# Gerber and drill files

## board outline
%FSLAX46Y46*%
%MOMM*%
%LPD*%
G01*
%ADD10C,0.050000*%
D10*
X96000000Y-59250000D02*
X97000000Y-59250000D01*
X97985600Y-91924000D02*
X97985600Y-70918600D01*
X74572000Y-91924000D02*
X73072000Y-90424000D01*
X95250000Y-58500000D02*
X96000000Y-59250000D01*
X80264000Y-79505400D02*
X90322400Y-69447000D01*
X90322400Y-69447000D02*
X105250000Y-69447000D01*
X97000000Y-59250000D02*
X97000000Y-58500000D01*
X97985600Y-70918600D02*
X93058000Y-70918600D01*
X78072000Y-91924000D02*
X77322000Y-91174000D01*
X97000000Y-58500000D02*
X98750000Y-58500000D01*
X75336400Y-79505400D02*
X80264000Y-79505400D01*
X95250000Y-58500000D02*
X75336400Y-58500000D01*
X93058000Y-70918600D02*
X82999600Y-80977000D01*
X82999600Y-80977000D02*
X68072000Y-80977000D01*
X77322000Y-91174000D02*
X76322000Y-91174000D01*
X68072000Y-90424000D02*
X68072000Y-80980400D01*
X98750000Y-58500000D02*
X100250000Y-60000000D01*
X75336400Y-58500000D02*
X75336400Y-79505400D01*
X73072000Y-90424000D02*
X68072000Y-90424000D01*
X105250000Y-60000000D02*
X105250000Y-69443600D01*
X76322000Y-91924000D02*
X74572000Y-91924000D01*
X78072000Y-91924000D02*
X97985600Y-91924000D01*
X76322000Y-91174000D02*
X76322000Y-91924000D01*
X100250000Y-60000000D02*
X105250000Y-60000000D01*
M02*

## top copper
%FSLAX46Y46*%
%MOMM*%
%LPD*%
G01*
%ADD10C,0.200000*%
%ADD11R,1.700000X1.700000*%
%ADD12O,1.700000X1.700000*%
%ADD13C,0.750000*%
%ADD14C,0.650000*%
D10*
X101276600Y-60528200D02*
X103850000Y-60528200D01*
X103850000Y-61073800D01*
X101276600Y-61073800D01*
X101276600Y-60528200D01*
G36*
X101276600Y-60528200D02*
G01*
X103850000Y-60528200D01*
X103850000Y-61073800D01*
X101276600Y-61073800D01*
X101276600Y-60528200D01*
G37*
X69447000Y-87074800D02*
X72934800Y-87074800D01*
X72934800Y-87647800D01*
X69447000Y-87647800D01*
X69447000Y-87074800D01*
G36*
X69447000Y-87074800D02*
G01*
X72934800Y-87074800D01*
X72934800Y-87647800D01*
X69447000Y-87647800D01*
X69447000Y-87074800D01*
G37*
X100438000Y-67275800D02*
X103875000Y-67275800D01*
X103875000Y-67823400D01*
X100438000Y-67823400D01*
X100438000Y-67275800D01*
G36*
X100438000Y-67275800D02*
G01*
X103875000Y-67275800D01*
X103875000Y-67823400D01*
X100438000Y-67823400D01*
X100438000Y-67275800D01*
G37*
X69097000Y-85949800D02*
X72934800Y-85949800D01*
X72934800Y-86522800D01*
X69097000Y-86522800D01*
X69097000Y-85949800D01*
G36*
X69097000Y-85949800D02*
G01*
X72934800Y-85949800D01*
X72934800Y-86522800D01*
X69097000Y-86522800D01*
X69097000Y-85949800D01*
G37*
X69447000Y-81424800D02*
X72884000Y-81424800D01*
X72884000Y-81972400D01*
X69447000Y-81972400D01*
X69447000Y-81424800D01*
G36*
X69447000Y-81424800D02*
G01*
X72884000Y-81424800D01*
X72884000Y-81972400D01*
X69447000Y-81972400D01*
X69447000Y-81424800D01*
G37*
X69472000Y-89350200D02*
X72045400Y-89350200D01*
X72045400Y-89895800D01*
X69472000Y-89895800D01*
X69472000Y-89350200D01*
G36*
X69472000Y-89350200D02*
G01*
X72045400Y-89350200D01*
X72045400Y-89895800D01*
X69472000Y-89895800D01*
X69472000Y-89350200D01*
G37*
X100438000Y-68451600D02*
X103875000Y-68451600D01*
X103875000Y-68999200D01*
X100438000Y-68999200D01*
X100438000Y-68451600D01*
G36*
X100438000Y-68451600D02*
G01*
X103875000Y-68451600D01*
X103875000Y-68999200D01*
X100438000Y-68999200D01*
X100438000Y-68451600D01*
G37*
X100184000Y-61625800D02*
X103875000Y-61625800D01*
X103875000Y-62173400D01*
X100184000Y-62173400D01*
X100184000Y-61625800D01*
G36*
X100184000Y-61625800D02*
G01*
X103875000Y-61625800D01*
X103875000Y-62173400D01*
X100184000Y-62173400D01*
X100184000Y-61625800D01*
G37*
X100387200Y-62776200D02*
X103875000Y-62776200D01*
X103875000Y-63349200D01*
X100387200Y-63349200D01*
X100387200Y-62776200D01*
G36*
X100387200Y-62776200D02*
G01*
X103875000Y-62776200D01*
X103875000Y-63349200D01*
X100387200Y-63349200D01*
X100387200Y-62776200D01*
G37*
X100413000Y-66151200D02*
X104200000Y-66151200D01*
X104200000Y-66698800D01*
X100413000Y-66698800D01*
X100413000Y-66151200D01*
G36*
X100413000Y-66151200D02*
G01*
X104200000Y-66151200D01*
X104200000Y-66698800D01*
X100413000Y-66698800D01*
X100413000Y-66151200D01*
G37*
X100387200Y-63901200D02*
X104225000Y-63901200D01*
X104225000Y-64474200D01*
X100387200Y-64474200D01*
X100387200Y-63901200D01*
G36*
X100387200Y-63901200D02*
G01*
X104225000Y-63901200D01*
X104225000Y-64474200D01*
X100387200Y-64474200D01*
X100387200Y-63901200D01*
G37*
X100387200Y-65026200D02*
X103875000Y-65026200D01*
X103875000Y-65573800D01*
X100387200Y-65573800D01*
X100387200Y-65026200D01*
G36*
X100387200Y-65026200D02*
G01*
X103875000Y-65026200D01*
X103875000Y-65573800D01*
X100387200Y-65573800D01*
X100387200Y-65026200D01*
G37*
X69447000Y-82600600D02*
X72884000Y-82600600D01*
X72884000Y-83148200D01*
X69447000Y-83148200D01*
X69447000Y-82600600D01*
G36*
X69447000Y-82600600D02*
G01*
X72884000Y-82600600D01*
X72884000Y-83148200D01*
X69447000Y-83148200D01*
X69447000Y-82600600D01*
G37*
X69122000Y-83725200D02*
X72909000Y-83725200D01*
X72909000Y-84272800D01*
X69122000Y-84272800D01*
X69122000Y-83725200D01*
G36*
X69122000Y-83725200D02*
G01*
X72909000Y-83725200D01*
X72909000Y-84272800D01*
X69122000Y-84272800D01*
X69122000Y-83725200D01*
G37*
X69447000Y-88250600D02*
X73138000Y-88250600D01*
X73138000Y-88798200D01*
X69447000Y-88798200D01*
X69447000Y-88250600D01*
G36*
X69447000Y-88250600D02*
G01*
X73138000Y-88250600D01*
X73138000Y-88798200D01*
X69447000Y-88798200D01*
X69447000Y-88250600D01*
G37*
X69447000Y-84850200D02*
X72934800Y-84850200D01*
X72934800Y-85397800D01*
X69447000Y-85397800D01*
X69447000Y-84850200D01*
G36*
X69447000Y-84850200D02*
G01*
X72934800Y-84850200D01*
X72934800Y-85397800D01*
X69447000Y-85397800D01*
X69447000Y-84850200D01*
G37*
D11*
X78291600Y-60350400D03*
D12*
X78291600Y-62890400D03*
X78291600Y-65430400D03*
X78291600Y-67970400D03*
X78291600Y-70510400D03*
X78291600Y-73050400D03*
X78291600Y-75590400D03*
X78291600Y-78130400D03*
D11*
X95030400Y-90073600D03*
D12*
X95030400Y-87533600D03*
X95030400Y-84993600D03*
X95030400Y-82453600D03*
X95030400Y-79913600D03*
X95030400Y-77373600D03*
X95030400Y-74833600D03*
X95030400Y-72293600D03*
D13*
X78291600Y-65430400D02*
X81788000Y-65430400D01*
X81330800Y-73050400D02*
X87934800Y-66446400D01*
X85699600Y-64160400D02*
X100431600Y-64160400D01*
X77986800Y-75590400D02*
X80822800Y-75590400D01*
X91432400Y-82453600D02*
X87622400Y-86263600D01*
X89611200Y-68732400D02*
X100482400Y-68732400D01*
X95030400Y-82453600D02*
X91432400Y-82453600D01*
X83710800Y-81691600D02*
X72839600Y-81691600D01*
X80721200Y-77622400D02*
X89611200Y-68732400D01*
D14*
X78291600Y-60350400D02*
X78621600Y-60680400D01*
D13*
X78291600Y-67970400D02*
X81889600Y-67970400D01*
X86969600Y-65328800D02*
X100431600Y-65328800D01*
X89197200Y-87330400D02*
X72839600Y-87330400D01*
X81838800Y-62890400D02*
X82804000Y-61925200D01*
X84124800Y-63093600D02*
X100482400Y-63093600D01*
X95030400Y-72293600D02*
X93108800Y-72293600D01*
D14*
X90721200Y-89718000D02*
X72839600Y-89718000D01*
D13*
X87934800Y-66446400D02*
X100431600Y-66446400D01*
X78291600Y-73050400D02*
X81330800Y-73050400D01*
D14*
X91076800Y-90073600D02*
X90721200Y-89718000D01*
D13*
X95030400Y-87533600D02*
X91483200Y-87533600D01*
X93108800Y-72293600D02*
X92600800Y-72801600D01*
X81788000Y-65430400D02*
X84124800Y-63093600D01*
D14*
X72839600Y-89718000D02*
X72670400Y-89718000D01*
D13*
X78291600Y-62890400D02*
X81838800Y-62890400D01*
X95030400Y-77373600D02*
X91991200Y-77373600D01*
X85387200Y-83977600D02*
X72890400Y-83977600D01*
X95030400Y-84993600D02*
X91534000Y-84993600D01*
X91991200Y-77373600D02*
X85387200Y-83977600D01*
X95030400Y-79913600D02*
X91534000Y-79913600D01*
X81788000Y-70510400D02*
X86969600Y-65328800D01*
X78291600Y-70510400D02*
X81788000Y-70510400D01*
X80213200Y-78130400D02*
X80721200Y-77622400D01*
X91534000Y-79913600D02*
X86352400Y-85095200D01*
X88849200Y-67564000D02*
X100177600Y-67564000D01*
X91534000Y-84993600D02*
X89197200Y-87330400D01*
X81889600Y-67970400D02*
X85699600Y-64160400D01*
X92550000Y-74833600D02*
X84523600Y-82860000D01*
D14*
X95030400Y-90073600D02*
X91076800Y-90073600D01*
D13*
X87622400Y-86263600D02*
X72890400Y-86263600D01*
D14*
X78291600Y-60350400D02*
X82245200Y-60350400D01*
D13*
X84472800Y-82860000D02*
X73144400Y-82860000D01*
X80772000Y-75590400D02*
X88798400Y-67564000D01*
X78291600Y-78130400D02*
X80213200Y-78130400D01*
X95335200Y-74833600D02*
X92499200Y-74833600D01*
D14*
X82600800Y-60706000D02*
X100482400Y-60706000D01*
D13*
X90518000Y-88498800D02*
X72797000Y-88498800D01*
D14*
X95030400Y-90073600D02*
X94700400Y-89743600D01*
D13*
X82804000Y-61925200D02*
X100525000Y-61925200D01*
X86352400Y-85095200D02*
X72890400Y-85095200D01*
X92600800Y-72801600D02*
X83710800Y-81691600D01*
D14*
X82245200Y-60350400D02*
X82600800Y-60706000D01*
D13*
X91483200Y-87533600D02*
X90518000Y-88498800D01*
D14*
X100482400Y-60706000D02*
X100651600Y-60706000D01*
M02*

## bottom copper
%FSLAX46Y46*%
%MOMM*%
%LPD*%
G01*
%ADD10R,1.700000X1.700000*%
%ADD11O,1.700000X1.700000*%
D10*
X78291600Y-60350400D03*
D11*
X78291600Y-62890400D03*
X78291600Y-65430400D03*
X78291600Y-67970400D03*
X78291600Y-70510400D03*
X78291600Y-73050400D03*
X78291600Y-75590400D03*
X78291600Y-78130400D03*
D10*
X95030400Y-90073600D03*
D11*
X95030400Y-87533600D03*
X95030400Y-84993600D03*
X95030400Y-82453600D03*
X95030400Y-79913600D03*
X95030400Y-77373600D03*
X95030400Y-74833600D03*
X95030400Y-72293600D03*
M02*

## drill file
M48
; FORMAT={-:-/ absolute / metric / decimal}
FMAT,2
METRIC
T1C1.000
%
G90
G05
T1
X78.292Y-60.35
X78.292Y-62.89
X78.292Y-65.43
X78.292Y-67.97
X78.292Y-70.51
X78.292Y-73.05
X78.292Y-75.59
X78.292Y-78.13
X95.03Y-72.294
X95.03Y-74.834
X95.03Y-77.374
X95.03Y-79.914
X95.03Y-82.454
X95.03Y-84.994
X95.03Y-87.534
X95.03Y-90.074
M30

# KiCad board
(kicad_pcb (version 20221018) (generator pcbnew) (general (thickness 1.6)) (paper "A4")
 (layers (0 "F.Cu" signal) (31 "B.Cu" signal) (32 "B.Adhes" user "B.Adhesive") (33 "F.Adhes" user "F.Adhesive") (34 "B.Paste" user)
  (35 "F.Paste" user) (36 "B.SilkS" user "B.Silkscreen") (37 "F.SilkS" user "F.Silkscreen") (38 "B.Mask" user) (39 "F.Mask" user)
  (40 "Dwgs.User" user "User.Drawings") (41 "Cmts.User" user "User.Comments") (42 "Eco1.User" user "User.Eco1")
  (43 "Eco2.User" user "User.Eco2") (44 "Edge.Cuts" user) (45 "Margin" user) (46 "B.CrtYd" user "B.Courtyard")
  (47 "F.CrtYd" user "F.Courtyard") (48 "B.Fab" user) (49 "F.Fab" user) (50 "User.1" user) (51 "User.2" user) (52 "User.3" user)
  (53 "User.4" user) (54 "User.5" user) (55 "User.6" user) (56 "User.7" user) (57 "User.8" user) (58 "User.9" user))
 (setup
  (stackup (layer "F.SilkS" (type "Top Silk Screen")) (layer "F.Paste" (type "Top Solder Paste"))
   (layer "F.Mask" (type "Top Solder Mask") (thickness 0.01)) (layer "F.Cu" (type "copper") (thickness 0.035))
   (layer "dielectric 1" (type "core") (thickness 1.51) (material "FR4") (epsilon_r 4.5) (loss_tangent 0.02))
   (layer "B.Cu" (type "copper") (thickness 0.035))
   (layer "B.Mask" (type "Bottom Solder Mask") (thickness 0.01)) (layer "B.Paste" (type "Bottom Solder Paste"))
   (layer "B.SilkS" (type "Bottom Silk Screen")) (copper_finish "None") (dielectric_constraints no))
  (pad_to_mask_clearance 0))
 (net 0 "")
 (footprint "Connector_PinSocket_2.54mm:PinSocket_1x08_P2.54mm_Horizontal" (layer "F.Cu") (at 78.2916 60.3504)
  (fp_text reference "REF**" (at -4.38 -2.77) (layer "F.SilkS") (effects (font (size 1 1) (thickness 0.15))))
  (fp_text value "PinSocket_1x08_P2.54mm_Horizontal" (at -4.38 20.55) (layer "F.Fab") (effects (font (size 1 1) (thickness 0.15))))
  (pad "1" thru_hole rect (at 0 0) (size 1.7 1.7) (drill 1) (layers "*.Cu" "*.Mask"))
  (pad "2" thru_hole oval (at 0 2.54) (size 1.7 1.7) (drill 1) (layers "*.Cu" "*.Mask"))
  (pad "3" thru_hole oval (at 0 5.08) (size 1.7 1.7) (drill 1) (layers "*.Cu" "*.Mask"))
  (pad "4" thru_hole oval (at 0 7.62) (size 1.7 1.7) (drill 1) (layers "*.Cu" "*.Mask"))
  (pad "5" thru_hole oval (at 0 10.16) (size 1.7 1.7) (drill 1) (layers "*.Cu" "*.Mask"))
  (pad "6" thru_hole oval (at 0 12.7) (size 1.7 1.7) (drill 1) (layers "*.Cu" "*.Mask"))
  (pad "7" thru_hole oval (at 0 15.24) (size 1.7 1.7) (drill 1) (layers "*.Cu" "*.Mask"))
  (pad "8" thru_hole oval (at 0 17.78) (size 1.7 1.7) (drill 1) (layers "*.Cu" "*.Mask")))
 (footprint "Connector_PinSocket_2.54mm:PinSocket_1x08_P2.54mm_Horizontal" (layer "F.Cu") (at 95.0304 90.0736 180)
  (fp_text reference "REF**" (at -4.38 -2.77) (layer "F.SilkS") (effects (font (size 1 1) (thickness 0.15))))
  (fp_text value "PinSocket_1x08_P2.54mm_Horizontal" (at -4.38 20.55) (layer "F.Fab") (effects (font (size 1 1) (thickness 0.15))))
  (pad "1" thru_hole rect (at 0 0 180) (size 1.7 1.7) (drill 1) (layers "*.Cu" "*.Mask"))
  (pad "2" thru_hole oval (at 0 2.54 180) (size 1.7 1.7) (drill 1) (layers "*.Cu" "*.Mask"))
  (pad "3" thru_hole oval (at 0 5.08 180) (size 1.7 1.7) (drill 1) (layers "*.Cu" "*.Mask"))
  (pad "4" thru_hole oval (at 0 7.62 180) (size 1.7 1.7) (drill 1) (layers "*.Cu" "*.Mask"))
  (pad "5" thru_hole oval (at 0 10.16 180) (size 1.7 1.7) (drill 1) (layers "*.Cu" "*.Mask"))
  (pad "6" thru_hole oval (at 0 12.7 180) (size 1.7 1.7) (drill 1) (layers "*.Cu" "*.Mask"))
  (pad "7" thru_hole oval (at 0 15.24 180) (size 1.7 1.7) (drill 1) (layers "*.Cu" "*.Mask"))
  (pad "8" thru_hole oval (at 0 17.78 180) (size 1.7 1.7) (drill 1) (layers "*.Cu" "*.Mask")))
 (gr_rect (start 101.2766 60.5282) (end 103.85 61.0738) (stroke (width 0.2) (type solid)) (fill solid) (layer "F.Cu"))
 (gr_rect (start 72.9348 87.6478) (end 69.447 87.0748) (stroke (width 0.2) (type solid)) (fill solid) (layer "F.Cu"))
 (gr_rect (start 100.438 67.2758) (end 103.875 67.8234) (stroke (width 0.2) (type solid)) (fill solid) (layer "F.Cu"))
 (gr_rect (start 72.9348 86.5228) (end 69.097 85.9498) (stroke (width 0.2) (type solid)) (fill solid) (layer "F.Cu"))
 (gr_rect (start 72.884 81.9724) (end 69.447 81.4248) (stroke (width 0.2) (type solid)) (fill solid) (layer "F.Cu"))
 (gr_rect (start 72.0454 89.8958) (end 69.472 89.3502) (stroke (width 0.2) (type solid)) (fill solid) (layer "F.Cu"))
 (gr_rect (start 100.438 68.4516) (end 103.875 68.9992) (stroke (width 0.2) (type solid)) (fill solid) (layer "F.Cu"))
 (gr_rect (start 100.184 61.6258) (end 103.875 62.1734) (stroke (width 0.2) (type solid)) (fill solid) (layer "F.Cu"))
 (gr_rect (start 100.3872 62.7762) (end 103.875 63.3492) (stroke (width 0.2) (type solid)) (fill solid) (layer "F.Cu"))
 (gr_rect (start 100.413 66.1512) (end 104.2 66.6988) (stroke (width 0.2) (type solid)) (fill solid) (layer "F.Cu"))
 (gr_rect (start 100.3872 63.9012) (end 104.225 64.4742) (stroke (width 0.2) (type solid)) (fill solid) (layer "F.Cu"))
 (gr_rect (start 100.3872 65.0262) (end 103.875 65.5738) (stroke (width 0.2) (type solid)) (fill solid) (layer "F.Cu"))
 (gr_rect (start 72.884 83.1482) (end 69.447 82.6006) (stroke (width 0.2) (type solid)) (fill solid) (layer "F.Cu"))
 (gr_rect (start 72.909 84.2728) (end 69.122 83.7252) (stroke (width 0.2) (type solid)) (fill solid) (layer "F.Cu"))
 (gr_rect (start 73.138 88.7982) (end 69.447 88.2506) (stroke (width 0.2) (type solid)) (fill solid) (layer "F.Cu"))
 (gr_rect (start 72.9348 85.3978) (end 69.447 84.8502) (stroke (width 0.2) (type solid)) (fill solid) (layer "F.Cu"))
 (gr_line (start 96 59.25) (end 97 59.25) (stroke (width 0.05) (type default)) (layer "Edge.Cuts"))
 (gr_line (start 97.9856 91.924) (end 97.9856 70.9186) (stroke (width 0.05) (type default)) (layer "Edge.Cuts"))
 (gr_line (start 74.572 91.924) (end 73.072 90.424) (stroke (width 0.05) (type default)) (layer "Edge.Cuts"))
 (gr_line (start 95.25 58.5) (end 96 59.25) (stroke (width 0.05) (type default)) (layer "Edge.Cuts"))
 (gr_line (start 80.264 79.5054) (end 90.3224 69.447) (stroke (width 0.05) (type default)) (layer "Edge.Cuts"))
 (gr_line (start 90.3224 69.447) (end 105.25 69.447) (stroke (width 0.05) (type default)) (layer "Edge.Cuts"))
 (gr_line (start 97 59.25) (end 97 58.5) (stroke (width 0.05) (type default)) (layer "Edge.Cuts"))
 (gr_line (start 97.9856 70.9186) (end 93.058 70.9186) (stroke (width 0.05) (type default)) (layer "Edge.Cuts"))
 (gr_line (start 78.072 91.924) (end 77.322 91.174) (stroke (width 0.05) (type default)) (layer "Edge.Cuts"))
 (gr_line (start 97 58.5) (end 98.75 58.5) (stroke (width 0.05) (type default)) (layer "Edge.Cuts"))
 (gr_line (start 75.3364 79.5054) (end 80.264 79.5054) (stroke (width 0.05) (type default)) (layer "Edge.Cuts"))
 (gr_line (start 95.25 58.5) (end 75.3364 58.5) (stroke (width 0.05) (type default)) (layer "Edge.Cuts"))
 (gr_line (start 93.058 70.9186) (end 82.9996 80.977) (stroke (width 0.05) (type default)) (layer "Edge.Cuts"))
 (gr_line (start 82.9996 80.977) (end 68.072 80.977) (stroke (width 0.05) (type default)) (layer "Edge.Cuts"))
 (gr_line (start 77.322 91.174) (end 76.322 91.174) (stroke (width 0.05) (type default)) (layer "Edge.Cuts"))
 (gr_line (start 68.072 90.424) (end 68.072 80.9804) (stroke (width 0.05) (type default)) (layer "Edge.Cuts"))
 (gr_line (start 98.75 58.5) (end 100.25 60) (stroke (width 0.05) (type default)) (layer "Edge.Cuts"))
 (gr_line (start 75.3364 58.5) (end 75.3364 79.5054) (stroke (width 0.05) (type default)) (layer "Edge.Cuts"))
 (gr_line (start 73.072 90.424) (end 68.072 90.424) (stroke (width 0.05) (type default)) (layer "Edge.Cuts"))
 (gr_line (start 105.25 60) (end 105.25 69.4436) (stroke (width 0.05) (type default)) (layer "Edge.Cuts"))
 (gr_line (start 76.322 91.924) (end 74.572 91.924) (stroke (width 0.05) (type default)) (layer "Edge.Cuts"))
 (gr_line (start 78.072 91.924) (end 97.9856 91.924) (stroke (width 0.05) (type default)) (layer "Edge.Cuts"))
 (gr_line (start 76.322 91.174) (end 76.322 91.924) (stroke (width 0.05) (type default)) (layer "Edge.Cuts"))
 (gr_line (start 100.25 60) (end 105.25 60) (stroke (width 0.05) (type default)) (layer "Edge.Cuts"))
 (segment (start 78.2916 65.4304) (end 81.788 65.4304) (width 0.75) (layer "F.Cu") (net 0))
 (segment (start 81.3308 73.0504) (end 87.9348 66.4464) (width 0.75) (layer "F.Cu") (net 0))
 (segment (start 85.6996 64.1604) (end 100.4316 64.1604) (width 0.75) (layer "F.Cu") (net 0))
 (segment (start 77.9868 75.5904) (end 80.8228 75.5904) (width 0.75) (layer "F.Cu") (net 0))
 (segment (start 91.4324 82.4536) (end 87.6224 86.2636) (width 0.75) (layer "F.Cu") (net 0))
 (segment (start 89.6112 68.7324) (end 100.4824 68.7324) (width 0.75) (layer "F.Cu") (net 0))
 (segment (start 95.0304 82.4536) (end 91.4324 82.4536) (width 0.75) (layer "F.Cu") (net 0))
 (segment (start 83.7108 81.6916) (end 72.8396 81.6916) (width 0.75) (layer "F.Cu") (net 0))
 (segment (start 80.7212 77.6224) (end 89.6112 68.7324) (width 0.75) (layer "F.Cu") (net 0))
 (segment (start 78.2916 60.3504) (end 78.6216 60.6804) (width 0.65) (layer "F.Cu") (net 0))
 (segment (start 78.2916 67.9704) (end 81.8896 67.9704) (width 0.75) (layer "F.Cu") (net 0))
 (segment (start 86.9696 65.3288) (end 100.4316 65.3288) (width 0.75) (layer "F.Cu") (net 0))
 (segment (start 89.1972 87.3304) (end 72.8396 87.3304) (width 0.75) (layer "F.Cu") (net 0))
 (segment (start 81.8388 62.8904) (end 82.804 61.9252) (width 0.75) (layer "F.Cu") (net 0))
 (segment (start 84.1248 63.0936) (end 100.4824 63.0936) (width 0.75) (layer "F.Cu") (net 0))
 (segment (start 95.0304 72.2936) (end 93.1088 72.2936) (width 0.75) (layer "F.Cu") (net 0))
 (segment (start 90.7212 89.718) (end 72.8396 89.718) (width 0.65) (layer "F.Cu") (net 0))
 (segment (start 87.9348 66.4464) (end 100.4316 66.4464) (width 0.75) (layer "F.Cu") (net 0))
 (segment (start 78.2916 73.0504) (end 81.3308 73.0504) (width 0.75) (layer "F.Cu") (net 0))
 (segment (start 91.0768 90.0736) (end 90.7212 89.718) (width 0.65) (layer "F.Cu") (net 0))
 (segment (start 95.0304 87.5336) (end 91.4832 87.5336) (width 0.75) (layer "F.Cu") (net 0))
 (segment (start 93.1088 72.2936) (end 92.6008 72.8016) (width 0.75) (layer "F.Cu") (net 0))
 (segment (start 81.788 65.4304) (end 84.1248 63.0936) (width 0.75) (layer "F.Cu") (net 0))
 (segment (start 72.8396 89.718) (end 72.6704 89.718) (width 0.65) (layer "F.Cu") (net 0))
 (segment (start 78.2916 62.8904) (end 81.8388 62.8904) (width 0.75) (layer "F.Cu") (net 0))
 (segment (start 95.0304 77.3736) (end 91.9912 77.3736) (width 0.75) (layer "F.Cu") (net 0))
 (segment (start 85.3872 83.9776) (end 72.8904 83.9776) (width 0.75) (layer "F.Cu") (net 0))
 (segment (start 95.0304 84.9936) (end 91.534 84.9936) (width 0.75) (layer "F.Cu") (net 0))
 (segment (start 91.9912 77.3736) (end 85.3872 83.9776) (width 0.75) (layer "F.Cu") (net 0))
 (segment (start 95.0304 79.9136) (end 91.534 79.9136) (width 0.75) (layer "F.Cu") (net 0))
 (segment (start 81.788 70.5104) (end 86.9696 65.3288) (width 0.75) (layer "F.Cu") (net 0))
 (segment (start 78.2916 70.5104) (end 81.788 70.5104) (width 0.75) (layer "F.Cu") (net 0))
 (segment (start 80.2132 78.1304) (end 80.7212 77.6224) (width 0.75) (layer "F.Cu") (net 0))
 (segment (start 91.534 79.9136) (end 86.3524 85.0952) (width 0.75) (layer "F.Cu") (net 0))
 (segment (start 88.8492 67.564) (end 100.1776 67.564) (width 0.75) (layer "F.Cu") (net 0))
 (segment (start 91.534 84.9936) (end 89.1972 87.3304) (width 0.75) (layer "F.Cu") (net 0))
 (segment (start 81.8896 67.9704) (end 85.6996 64.1604) (width 0.75) (layer "F.Cu") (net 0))
 (segment (start 92.55 74.8336) (end 84.5236 82.86) (width 0.75) (layer "F.Cu") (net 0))
 (segment (start 95.0304 90.0736) (end 91.0768 90.0736) (width 0.65) (layer "F.Cu") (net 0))
 (segment (start 87.6224 86.2636) (end 72.8904 86.2636) (width 0.75) (layer "F.Cu") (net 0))
 (segment (start 78.2916 60.3504) (end 82.2452 60.3504) (width 0.65) (layer "F.Cu") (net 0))
 (segment (start 84.4728 82.86) (end 73.1444 82.86) (width 0.75) (layer "F.Cu") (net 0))
 (segment (start 80.772 75.5904) (end 88.7984 67.564) (width 0.75) (layer "F.Cu") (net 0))
 (segment (start 78.2916 78.1304) (end 80.2132 78.1304) (width 0.75) (layer "F.Cu") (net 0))
 (segment (start 95.3352 74.8336) (end 92.4992 74.8336) (width 0.75) (layer "F.Cu") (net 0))
 (segment (start 82.6008 60.706) (end 100.4824 60.706) (width 0.65) (layer "F.Cu") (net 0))
 (segment (start 90.518 88.4988) (end 72.797 88.4988) (width 0.75) (layer "F.Cu") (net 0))
 (segment (start 95.0304 90.0736) (end 94.7004 89.7436) (width 0.65) (layer "F.Cu") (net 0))
 (segment (start 82.804 61.9252) (end 100.525 61.9252) (width 0.75) (layer "F.Cu") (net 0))
 (segment (start 86.3524 85.0952) (end 72.8904 85.0952) (width 0.75) (layer "F.Cu") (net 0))
 (segment (start 92.6008 72.8016) (end 83.7108 81.6916) (width 0.75) (layer "F.Cu") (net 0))
 (segment (start 82.2452 60.3504) (end 82.6008 60.706) (width 0.65) (layer "F.Cu") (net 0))
 (segment (start 91.4832 87.5336) (end 90.518 88.4988) (width 0.75) (layer "F.Cu") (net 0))
 (segment (start 100.4824 60.706) (end 100.6516 60.706) (width 0.65) (layer "F.Cu") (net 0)))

